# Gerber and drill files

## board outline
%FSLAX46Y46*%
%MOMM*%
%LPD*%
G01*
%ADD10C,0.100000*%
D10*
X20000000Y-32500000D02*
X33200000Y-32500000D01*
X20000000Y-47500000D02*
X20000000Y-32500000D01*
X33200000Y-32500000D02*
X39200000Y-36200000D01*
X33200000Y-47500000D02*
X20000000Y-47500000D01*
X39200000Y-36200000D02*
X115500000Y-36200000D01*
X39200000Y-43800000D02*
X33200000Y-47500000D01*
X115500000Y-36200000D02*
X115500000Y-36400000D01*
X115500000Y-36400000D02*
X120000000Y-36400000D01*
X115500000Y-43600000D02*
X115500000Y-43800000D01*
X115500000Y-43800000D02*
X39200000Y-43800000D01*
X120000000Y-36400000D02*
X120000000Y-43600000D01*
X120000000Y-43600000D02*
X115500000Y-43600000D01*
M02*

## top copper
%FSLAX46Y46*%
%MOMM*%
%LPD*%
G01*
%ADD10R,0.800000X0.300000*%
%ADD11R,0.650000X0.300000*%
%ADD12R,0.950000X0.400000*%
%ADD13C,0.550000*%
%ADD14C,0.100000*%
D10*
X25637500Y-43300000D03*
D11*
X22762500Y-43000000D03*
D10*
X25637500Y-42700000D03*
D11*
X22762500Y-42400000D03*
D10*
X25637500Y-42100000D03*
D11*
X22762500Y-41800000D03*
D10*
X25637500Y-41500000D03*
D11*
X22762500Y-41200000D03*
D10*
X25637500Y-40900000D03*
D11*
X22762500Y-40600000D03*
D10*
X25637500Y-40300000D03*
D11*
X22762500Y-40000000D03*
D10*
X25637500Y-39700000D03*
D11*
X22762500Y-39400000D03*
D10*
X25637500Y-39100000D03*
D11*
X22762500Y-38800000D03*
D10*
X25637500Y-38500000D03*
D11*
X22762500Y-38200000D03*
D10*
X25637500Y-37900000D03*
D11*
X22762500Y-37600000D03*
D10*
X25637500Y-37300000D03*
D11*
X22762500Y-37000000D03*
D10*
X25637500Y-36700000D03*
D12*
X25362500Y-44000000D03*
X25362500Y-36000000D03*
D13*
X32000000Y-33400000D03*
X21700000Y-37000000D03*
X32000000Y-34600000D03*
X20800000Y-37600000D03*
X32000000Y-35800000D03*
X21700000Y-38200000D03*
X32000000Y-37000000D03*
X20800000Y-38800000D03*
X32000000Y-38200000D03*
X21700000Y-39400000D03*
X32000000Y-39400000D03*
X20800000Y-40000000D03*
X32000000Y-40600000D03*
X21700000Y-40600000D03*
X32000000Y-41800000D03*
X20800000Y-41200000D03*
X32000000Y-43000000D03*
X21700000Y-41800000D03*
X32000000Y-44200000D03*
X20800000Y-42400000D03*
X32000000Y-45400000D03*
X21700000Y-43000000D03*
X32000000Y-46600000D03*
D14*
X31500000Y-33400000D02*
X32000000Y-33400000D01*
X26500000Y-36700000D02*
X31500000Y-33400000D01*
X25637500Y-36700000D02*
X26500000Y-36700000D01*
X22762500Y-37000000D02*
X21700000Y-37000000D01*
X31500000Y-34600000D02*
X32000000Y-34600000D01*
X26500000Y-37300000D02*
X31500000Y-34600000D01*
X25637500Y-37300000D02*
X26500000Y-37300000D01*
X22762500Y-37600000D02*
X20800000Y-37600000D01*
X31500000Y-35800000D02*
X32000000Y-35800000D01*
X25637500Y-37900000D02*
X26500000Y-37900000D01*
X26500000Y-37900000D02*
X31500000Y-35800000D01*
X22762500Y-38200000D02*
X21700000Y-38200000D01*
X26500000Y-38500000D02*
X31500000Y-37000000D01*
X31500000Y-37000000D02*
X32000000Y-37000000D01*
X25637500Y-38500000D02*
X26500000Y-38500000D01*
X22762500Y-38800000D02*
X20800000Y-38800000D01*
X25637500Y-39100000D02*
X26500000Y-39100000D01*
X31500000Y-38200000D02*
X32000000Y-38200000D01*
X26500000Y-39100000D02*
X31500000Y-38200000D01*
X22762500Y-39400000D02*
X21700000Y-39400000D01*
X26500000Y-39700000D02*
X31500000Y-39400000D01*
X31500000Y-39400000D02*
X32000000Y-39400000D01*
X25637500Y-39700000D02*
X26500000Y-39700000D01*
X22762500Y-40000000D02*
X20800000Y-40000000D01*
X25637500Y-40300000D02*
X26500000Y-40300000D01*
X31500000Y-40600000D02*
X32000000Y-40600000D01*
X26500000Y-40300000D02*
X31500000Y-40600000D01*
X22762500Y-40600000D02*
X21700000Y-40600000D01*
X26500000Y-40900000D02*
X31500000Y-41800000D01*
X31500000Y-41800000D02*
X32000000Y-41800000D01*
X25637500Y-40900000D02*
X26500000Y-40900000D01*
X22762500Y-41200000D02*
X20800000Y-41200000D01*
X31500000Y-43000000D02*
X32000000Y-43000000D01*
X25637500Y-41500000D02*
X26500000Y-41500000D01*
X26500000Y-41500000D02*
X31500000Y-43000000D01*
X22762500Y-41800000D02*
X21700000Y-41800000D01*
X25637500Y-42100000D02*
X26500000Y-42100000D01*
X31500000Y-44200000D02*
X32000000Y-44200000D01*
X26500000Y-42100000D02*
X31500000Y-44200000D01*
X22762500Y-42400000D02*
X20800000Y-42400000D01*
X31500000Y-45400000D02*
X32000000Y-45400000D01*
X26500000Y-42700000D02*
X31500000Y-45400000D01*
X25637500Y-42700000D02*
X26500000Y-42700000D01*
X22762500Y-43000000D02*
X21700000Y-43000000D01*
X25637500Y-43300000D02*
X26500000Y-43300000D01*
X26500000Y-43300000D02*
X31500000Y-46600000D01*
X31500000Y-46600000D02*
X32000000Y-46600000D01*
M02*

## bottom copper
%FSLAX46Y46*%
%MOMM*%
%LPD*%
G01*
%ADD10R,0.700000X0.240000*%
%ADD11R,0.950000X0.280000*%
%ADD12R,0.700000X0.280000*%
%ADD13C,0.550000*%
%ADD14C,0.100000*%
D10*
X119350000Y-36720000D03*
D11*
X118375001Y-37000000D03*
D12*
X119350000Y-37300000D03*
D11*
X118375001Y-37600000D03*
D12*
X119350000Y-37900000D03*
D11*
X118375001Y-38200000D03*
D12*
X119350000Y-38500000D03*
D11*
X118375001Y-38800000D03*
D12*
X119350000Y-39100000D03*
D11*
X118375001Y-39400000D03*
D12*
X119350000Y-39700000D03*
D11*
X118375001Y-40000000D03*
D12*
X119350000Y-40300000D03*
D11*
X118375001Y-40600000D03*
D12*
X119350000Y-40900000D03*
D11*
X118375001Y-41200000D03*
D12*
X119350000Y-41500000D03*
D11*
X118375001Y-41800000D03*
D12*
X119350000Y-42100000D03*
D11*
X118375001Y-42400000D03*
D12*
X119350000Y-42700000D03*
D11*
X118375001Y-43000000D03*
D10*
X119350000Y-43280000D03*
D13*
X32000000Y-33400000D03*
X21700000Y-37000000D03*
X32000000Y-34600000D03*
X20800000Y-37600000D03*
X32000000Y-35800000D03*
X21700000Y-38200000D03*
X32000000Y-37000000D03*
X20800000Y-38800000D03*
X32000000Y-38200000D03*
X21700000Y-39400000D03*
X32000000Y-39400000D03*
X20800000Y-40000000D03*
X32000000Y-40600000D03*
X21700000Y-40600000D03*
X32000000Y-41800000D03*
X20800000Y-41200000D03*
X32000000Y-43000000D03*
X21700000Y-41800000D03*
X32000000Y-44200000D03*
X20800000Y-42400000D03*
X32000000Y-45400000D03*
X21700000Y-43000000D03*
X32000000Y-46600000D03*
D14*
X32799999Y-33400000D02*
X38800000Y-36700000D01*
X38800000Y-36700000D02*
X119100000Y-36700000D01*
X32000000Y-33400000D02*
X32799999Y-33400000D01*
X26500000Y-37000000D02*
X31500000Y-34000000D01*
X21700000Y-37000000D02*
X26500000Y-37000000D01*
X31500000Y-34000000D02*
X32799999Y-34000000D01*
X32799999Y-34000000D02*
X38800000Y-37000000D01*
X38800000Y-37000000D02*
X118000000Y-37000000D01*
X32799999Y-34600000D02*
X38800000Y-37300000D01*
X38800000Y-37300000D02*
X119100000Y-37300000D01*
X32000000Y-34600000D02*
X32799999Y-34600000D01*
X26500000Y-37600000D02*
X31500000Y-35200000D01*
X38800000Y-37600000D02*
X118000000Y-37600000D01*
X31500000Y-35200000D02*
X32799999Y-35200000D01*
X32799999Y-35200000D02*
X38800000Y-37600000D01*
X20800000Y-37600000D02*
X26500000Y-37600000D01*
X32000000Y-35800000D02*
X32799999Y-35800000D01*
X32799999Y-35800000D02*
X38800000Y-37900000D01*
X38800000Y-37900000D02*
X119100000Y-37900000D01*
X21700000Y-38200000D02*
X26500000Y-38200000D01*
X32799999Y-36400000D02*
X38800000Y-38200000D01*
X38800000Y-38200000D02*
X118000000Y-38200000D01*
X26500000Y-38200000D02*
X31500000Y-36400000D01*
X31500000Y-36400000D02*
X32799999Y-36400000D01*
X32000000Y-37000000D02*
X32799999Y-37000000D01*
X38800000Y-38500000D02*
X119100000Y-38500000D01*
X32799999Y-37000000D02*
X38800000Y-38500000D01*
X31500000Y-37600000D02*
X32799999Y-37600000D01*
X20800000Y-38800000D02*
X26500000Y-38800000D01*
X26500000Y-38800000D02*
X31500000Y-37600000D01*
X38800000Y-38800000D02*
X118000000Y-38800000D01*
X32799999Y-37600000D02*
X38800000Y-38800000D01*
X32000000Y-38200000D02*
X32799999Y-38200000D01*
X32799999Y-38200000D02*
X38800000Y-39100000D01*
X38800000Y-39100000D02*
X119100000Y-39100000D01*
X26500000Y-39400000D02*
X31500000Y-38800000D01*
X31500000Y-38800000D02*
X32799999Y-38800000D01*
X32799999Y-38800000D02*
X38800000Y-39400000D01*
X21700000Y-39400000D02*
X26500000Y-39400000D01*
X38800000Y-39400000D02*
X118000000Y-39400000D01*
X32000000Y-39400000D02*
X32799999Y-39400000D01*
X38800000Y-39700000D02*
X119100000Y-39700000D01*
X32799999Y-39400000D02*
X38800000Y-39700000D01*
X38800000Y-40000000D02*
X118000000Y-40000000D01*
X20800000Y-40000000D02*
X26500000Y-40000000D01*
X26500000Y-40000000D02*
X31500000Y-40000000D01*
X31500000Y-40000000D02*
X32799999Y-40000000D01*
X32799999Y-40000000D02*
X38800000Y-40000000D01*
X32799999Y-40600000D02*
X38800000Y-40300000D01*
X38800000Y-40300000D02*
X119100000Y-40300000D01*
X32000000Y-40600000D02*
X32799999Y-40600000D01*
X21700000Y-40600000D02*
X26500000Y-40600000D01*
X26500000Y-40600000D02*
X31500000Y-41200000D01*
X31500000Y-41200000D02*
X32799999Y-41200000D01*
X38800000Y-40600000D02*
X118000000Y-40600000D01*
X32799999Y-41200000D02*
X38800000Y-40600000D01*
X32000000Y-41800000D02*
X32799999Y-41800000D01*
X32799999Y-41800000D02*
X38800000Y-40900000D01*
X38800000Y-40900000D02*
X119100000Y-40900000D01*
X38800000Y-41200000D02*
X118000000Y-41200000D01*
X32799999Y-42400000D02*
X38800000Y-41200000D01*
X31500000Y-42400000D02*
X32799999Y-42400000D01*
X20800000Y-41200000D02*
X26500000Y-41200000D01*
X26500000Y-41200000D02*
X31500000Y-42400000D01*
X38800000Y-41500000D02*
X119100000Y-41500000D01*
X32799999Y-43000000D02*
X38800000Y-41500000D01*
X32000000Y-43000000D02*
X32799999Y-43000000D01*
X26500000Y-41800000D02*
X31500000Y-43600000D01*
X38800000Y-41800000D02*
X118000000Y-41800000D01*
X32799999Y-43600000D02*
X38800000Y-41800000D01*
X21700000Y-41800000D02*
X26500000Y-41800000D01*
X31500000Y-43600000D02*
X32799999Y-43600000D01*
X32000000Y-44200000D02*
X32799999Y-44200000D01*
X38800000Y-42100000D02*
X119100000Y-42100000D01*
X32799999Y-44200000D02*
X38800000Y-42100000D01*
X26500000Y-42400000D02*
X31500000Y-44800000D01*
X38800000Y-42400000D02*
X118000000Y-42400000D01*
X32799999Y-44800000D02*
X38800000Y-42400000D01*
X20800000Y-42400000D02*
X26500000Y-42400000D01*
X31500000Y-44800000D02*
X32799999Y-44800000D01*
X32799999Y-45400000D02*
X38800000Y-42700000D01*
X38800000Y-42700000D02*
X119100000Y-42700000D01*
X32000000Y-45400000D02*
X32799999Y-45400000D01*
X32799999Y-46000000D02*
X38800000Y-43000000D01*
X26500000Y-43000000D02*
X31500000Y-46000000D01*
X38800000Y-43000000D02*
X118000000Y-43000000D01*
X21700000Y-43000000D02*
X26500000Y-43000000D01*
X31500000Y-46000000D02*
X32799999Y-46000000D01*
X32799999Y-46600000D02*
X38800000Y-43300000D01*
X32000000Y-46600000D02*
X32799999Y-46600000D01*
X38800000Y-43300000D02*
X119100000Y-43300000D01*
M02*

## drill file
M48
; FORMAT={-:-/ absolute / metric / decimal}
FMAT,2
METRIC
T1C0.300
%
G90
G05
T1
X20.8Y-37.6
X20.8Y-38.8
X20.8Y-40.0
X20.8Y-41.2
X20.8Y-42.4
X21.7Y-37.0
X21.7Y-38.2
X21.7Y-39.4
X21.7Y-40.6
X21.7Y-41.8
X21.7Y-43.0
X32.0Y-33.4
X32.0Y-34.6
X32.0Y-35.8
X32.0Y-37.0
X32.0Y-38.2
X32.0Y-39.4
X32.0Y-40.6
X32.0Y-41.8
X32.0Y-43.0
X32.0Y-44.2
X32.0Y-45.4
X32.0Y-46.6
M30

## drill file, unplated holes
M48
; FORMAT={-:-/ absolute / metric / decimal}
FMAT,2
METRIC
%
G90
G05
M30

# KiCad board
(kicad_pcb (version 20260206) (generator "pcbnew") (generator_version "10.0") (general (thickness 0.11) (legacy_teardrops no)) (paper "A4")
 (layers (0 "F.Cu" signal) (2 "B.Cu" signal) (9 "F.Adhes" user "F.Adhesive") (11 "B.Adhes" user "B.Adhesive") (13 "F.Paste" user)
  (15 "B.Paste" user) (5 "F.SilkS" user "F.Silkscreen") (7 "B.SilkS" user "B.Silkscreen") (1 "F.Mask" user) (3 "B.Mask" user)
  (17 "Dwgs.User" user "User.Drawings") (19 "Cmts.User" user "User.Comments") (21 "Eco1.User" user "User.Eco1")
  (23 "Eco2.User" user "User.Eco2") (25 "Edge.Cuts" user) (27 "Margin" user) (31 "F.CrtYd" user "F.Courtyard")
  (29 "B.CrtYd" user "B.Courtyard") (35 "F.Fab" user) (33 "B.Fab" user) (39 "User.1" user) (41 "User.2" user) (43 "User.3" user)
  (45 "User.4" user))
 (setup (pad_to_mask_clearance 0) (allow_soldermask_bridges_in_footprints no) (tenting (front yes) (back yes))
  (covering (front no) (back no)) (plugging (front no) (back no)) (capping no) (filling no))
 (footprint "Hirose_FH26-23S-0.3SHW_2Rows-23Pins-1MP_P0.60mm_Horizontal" (layer "F.Cu") (at 24.2375 40 180)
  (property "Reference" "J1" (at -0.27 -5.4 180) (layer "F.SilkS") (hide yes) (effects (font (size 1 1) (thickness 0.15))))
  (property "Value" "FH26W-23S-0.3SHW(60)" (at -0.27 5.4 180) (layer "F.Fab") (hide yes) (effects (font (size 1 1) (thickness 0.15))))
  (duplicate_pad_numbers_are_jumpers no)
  (pad "1" smd rect (at -1.4 -3.3 180) (size 0.8 0.3) (layers "F.Cu" "F.Mask" "F.Paste") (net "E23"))
  (pad "2" smd rect (at 1.475 -3 180) (size 0.65 0.3) (layers "F.Cu" "F.Mask" "F.Paste") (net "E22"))
  (pad "3" smd rect (at -1.4 -2.7 180) (size 0.8 0.3) (layers "F.Cu" "F.Mask" "F.Paste") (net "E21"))
  (pad "4" smd rect (at 1.475 -2.4 180) (size 0.65 0.3) (layers "F.Cu" "F.Mask" "F.Paste") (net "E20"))
  (pad "5" smd rect (at -1.4 -2.1 180) (size 0.8 0.3) (layers "F.Cu" "F.Mask" "F.Paste") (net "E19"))
  (pad "6" smd rect (at 1.475 -1.8 180) (size 0.65 0.3) (layers "F.Cu" "F.Mask" "F.Paste") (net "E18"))
  (pad "7" smd rect (at -1.4 -1.5 180) (size 0.8 0.3) (layers "F.Cu" "F.Mask" "F.Paste") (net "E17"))
  (pad "8" smd rect (at 1.475 -1.2 180) (size 0.65 0.3) (layers "F.Cu" "F.Mask" "F.Paste") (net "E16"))
  (pad "9" smd rect (at -1.4 -0.9 180) (size 0.8 0.3) (layers "F.Cu" "F.Mask" "F.Paste") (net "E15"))
  (pad "10" smd rect (at 1.475 -0.6 180) (size 0.65 0.3) (layers "F.Cu" "F.Mask" "F.Paste") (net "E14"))
  (pad "11" smd rect (at -1.4 -0.3 180) (size 0.8 0.3) (layers "F.Cu" "F.Mask" "F.Paste") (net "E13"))
  (pad "12" smd rect (at 1.475 0 180) (size 0.65 0.3) (layers "F.Cu" "F.Mask" "F.Paste") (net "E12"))
  (pad "13" smd rect (at -1.4 0.3 180) (size 0.8 0.3) (layers "F.Cu" "F.Mask" "F.Paste") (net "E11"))
  (pad "14" smd rect (at 1.475 0.6 180) (size 0.65 0.3) (layers "F.Cu" "F.Mask" "F.Paste") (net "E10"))
  (pad "15" smd rect (at -1.4 0.9 180) (size 0.8 0.3) (layers "F.Cu" "F.Mask" "F.Paste") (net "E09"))
  (pad "16" smd rect (at 1.475 1.2 180) (size 0.65 0.3) (layers "F.Cu" "F.Mask" "F.Paste") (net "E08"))
  (pad "17" smd rect (at -1.4 1.5 180) (size 0.8 0.3) (layers "F.Cu" "F.Mask" "F.Paste") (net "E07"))
  (pad "18" smd rect (at 1.475 1.8 180) (size 0.65 0.3) (layers "F.Cu" "F.Mask" "F.Paste") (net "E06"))
  (pad "19" smd rect (at -1.4 2.1 180) (size 0.8 0.3) (layers "F.Cu" "F.Mask" "F.Paste") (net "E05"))
  (pad "20" smd rect (at 1.475 2.4 180) (size 0.65 0.3) (layers "F.Cu" "F.Mask" "F.Paste") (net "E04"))
  (pad "21" smd rect (at -1.4 2.7 180) (size 0.8 0.3) (layers "F.Cu" "F.Mask" "F.Paste") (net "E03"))
  (pad "22" smd rect (at 1.475 3 180) (size 0.65 0.3) (layers "F.Cu" "F.Mask" "F.Paste") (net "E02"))
  (pad "23" smd rect (at -1.4 3.3 180) (size 0.8 0.3) (layers "F.Cu" "F.Mask" "F.Paste") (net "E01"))
  (pad "MP" smd rect (at -1.125 -4 180) (size 0.95 0.4) (layers "F.Cu" "F.Mask" "F.Paste"))
  (pad "MP" smd rect (at -1.125 4 180) (size 0.95 0.4) (layers "F.Cu" "F.Mask" "F.Paste")))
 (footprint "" (layer "B.Cu") (at 118.6 40 180)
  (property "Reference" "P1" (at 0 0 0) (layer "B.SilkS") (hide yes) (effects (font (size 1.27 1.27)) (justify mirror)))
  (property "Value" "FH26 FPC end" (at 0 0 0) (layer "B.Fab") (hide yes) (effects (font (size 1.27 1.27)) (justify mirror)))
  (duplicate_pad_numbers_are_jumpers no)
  (pad "1" smd rect (at -0.75 3.28 180) (size 0.7 0.24) (layers "B.Cu" "B.Mask") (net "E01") (thermal_bridge_angle 45))
  (pad "2" smd rect (at 0.224999 3 180) (size 0.95 0.28) (layers "B.Cu" "B.Mask") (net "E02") (thermal_bridge_angle 45))
  (pad "3" smd rect (at -0.75 2.7 180) (size 0.7 0.28) (layers "B.Cu" "B.Mask") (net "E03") (thermal_bridge_angle 45))
  (pad "4" smd rect (at 0.224999 2.4 180) (size 0.95 0.28) (layers "B.Cu" "B.Mask") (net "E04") (thermal_bridge_angle 45))
  (pad "5" smd rect (at -0.75 2.1 180) (size 0.7 0.28) (layers "B.Cu" "B.Mask") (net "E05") (thermal_bridge_angle 45))
  (pad "6" smd rect (at 0.224999 1.8 180) (size 0.95 0.28) (layers "B.Cu" "B.Mask") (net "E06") (thermal_bridge_angle 45))
  (pad "7" smd rect (at -0.75 1.5 180) (size 0.7 0.28) (layers "B.Cu" "B.Mask") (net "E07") (thermal_bridge_angle 45))
  (pad "8" smd rect (at 0.224999 1.2 180) (size 0.95 0.28) (layers "B.Cu" "B.Mask") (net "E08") (thermal_bridge_angle 45))
  (pad "9" smd rect (at -0.75 0.9 180) (size 0.7 0.28) (layers "B.Cu" "B.Mask") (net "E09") (thermal_bridge_angle 45))
  (pad "10" smd rect (at 0.224999 0.6 180) (size 0.95 0.28) (layers "B.Cu" "B.Mask") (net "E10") (thermal_bridge_angle 45))
  (pad "11" smd rect (at -0.75 0.3 180) (size 0.7 0.28) (layers "B.Cu" "B.Mask") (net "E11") (thermal_bridge_angle 45))
  (pad "12" smd rect (at 0.224999 0 180) (size 0.95 0.28) (layers "B.Cu" "B.Mask") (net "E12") (thermal_bridge_angle 45))
  (pad "13" smd rect (at -0.75 -0.3 180) (size 0.7 0.28) (layers "B.Cu" "B.Mask") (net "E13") (thermal_bridge_angle 45))
  (pad "14" smd rect (at 0.224999 -0.6 180) (size 0.95 0.28) (layers "B.Cu" "B.Mask") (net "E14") (thermal_bridge_angle 45))
  (pad "15" smd rect (at -0.75 -0.9 180) (size 0.7 0.28) (layers "B.Cu" "B.Mask") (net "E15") (thermal_bridge_angle 45))
  (pad "16" smd rect (at 0.224999 -1.2 180) (size 0.95 0.28) (layers "B.Cu" "B.Mask") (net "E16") (thermal_bridge_angle 45))
  (pad "17" smd rect (at -0.75 -1.5 180) (size 0.7 0.28) (layers "B.Cu" "B.Mask") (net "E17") (thermal_bridge_angle 45))
  (pad "18" smd rect (at 0.224999 -1.8 180) (size 0.95 0.28) (layers "B.Cu" "B.Mask") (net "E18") (thermal_bridge_angle 45))
  (pad "19" smd rect (at -0.75 -2.1 180) (size 0.7 0.28) (layers "B.Cu" "B.Mask") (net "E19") (thermal_bridge_angle 45))
  (pad "20" smd rect (at 0.224999 -2.4 180) (size 0.95 0.28) (layers "B.Cu" "B.Mask") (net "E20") (thermal_bridge_angle 45))
  (pad "21" smd rect (at -0.75 -2.7 180) (size 0.7 0.28) (layers "B.Cu" "B.Mask") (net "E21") (thermal_bridge_angle 45))
  (pad "22" smd rect (at 0.224999 -3 180) (size 0.95 0.28) (layers "B.Cu" "B.Mask") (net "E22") (thermal_bridge_angle 45))
  (pad "23" smd rect (at -0.75 -3.28 180) (size 0.7 0.24) (layers "B.Cu" "B.Mask") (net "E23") (thermal_bridge_angle 45)))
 (gr_line (start 20 32.5) (end 33.2 32.5) (stroke (width 0.1) (type default)) (layer "Edge.Cuts"))
 (gr_line (start 20 47.5) (end 20 32.5) (stroke (width 0.1) (type default)) (layer "Edge.Cuts"))
 (gr_line (start 33.2 32.5) (end 39.2 36.2) (stroke (width 0.1) (type default)) (layer "Edge.Cuts"))
 (gr_line (start 33.2 47.5) (end 20 47.5) (stroke (width 0.1) (type default)) (layer "Edge.Cuts"))
 (gr_line (start 39.2 36.2) (end 115.5 36.2) (stroke (width 0.1) (type default)) (layer "Edge.Cuts"))
 (gr_line (start 39.2 43.8) (end 33.2 47.5) (stroke (width 0.1) (type default)) (layer "Edge.Cuts"))
 (gr_line (start 115.5 36.2) (end 115.5 36.4) (stroke (width 0.1) (type default)) (layer "Edge.Cuts"))
 (gr_line (start 115.5 36.4) (end 120 36.4) (stroke (width 0.1) (type default)) (layer "Edge.Cuts"))
 (gr_line (start 115.5 43.6) (end 115.5 43.8) (stroke (width 0.1) (type default)) (layer "Edge.Cuts"))
 (gr_line (start 115.5 43.8) (end 39.2 43.8) (stroke (width 0.1) (type default)) (layer "Edge.Cuts"))
 (gr_line (start 120 36.4) (end 120 43.6) (stroke (width 0.1) (type default)) (layer "Edge.Cuts"))
 (gr_line (start 120 43.6) (end 115.5 43.6) (stroke (width 0.1) (type default)) (layer "Edge.Cuts"))
 (segment (start 31.5 33.4) (end 32 33.4) (width 0.1) (layer "F.Cu") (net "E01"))
 (segment (start 26.5 36.7) (end 31.5 33.4) (width 0.1) (layer "F.Cu") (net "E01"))
 (segment (start 25.6375 36.7) (end 26.5 36.7) (width 0.1) (layer "F.Cu") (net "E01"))
 (via (at 32 33.4) (size 0.55) (drill 0.3) (layers "F.Cu" "B.Cu") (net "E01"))
 (segment (start 32.799999 33.4) (end 38.8 36.7) (width 0.1) (layer "B.Cu") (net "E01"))
 (segment (start 38.8 36.7) (end 119.1 36.7) (width 0.1) (layer "B.Cu") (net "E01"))
 (segment (start 32 33.4) (end 32.799999 33.4) (width 0.1) (layer "B.Cu") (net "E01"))
 (segment (start 22.7625 37) (end 21.7 37) (width 0.1) (layer "F.Cu") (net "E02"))
 (via (at 21.7 37) (size 0.55) (drill 0.3) (layers "F.Cu" "B.Cu") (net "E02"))
 (segment (start 26.5 37) (end 31.5 34) (width 0.1) (layer "B.Cu") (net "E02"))
 (segment (start 21.7 37) (end 26.5 37) (width 0.1) (layer "B.Cu") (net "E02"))
 (segment (start 31.5 34) (end 32.799999 34) (width 0.1) (layer "B.Cu") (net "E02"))
 (segment (start 32.799999 34) (end 38.8 37) (width 0.1) (layer "B.Cu") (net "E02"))
 (segment (start 38.8 37) (end 118 37) (width 0.1) (layer "B.Cu") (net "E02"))
 (segment (start 31.5 34.6) (end 32 34.6) (width 0.1) (layer "F.Cu") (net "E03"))
 (segment (start 26.5 37.3) (end 31.5 34.6) (width 0.1) (layer "F.Cu") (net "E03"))
 (segment (start 25.6375 37.3) (end 26.5 37.3) (width 0.1) (layer "F.Cu") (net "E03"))
 (via (at 32 34.6) (size 0.55) (drill 0.3) (layers "F.Cu" "B.Cu") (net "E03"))
 (segment (start 32.799999 34.6) (end 38.8 37.3) (width 0.1) (layer "B.Cu") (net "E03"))
 (segment (start 38.8 37.3) (end 119.1 37.3) (width 0.1) (layer "B.Cu") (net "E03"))
 (segment (start 32 34.6) (end 32.799999 34.6) (width 0.1) (layer "B.Cu") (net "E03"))
 (segment (start 22.7625 37.6) (end 20.8 37.6) (width 0.1) (layer "F.Cu") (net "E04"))
 (via (at 20.8 37.6) (size 0.55) (drill 0.3) (layers "F.Cu" "B.Cu") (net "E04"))
 (segment (start 26.5 37.6) (end 31.5 35.2) (width 0.1) (layer "B.Cu") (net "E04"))
 (segment (start 38.8 37.6) (end 118 37.6) (width 0.1) (layer "B.Cu") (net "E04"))
 (segment (start 31.5 35.2) (end 32.799999 35.2) (width 0.1) (layer "B.Cu") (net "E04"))
 (segment (start 32.799999 35.2) (end 38.8 37.6) (width 0.1) (layer "B.Cu") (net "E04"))
 (segment (start 20.8 37.6) (end 26.5 37.6) (width 0.1) (layer "B.Cu") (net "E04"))
 (segment (start 31.5 35.8) (end 32 35.8) (width 0.1) (layer "F.Cu") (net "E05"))
 (segment (start 25.6375 37.9) (end 26.5 37.9) (width 0.1) (layer "F.Cu") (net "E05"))
 (segment (start 26.5 37.9) (end 31.5 35.8) (width 0.1) (layer "F.Cu") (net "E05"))
 (via (at 32 35.8) (size 0.55) (drill 0.3) (layers "F.Cu" "B.Cu") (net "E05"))
 (segment (start 32 35.8) (end 32.799999 35.8) (width 0.1) (layer "B.Cu") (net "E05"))
 (segment (start 32.799999 35.8) (end 38.8 37.9) (width 0.1) (layer "B.Cu") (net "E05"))
 (segment (start 38.8 37.9) (end 119.1 37.9) (width 0.1) (layer "B.Cu") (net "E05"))
 (segment (start 22.7625 38.2) (end 21.7 38.2) (width 0.1) (layer "F.Cu") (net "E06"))
 (via (at 21.7 38.2) (size 0.55) (drill 0.3) (layers "F.Cu" "B.Cu") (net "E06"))
 (segment (start 21.7 38.2) (end 26.5 38.2) (width 0.1) (layer "B.Cu") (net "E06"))
 (segment (start 32.799999 36.4) (end 38.8 38.2) (width 0.1) (layer "B.Cu") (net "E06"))
 (segment (start 38.8 38.2) (end 118 38.2) (width 0.1) (layer "B.Cu") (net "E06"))
 (segment (start 26.5 38.2) (end 31.5 36.4) (width 0.1) (layer "B.Cu") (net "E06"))
 (segment (start 31.5 36.4) (end 32.799999 36.4) (width 0.1) (layer "B.Cu") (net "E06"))
 (segment (start 26.5 38.5) (end 31.5 37) (width 0.1) (layer "F.Cu") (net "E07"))
 (segment (start 31.5 37) (end 32 37) (width 0.1) (layer "F.Cu") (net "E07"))
 (segment (start 25.6375 38.5) (end 26.5 38.5) (width 0.1) (layer "F.Cu") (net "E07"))
 (via (at 32 37) (size 0.55) (drill 0.3) (layers "F.Cu" "B.Cu") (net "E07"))
 (segment (start 32 37) (end 32.799999 37) (width 0.1) (layer "B.Cu") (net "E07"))
 (segment (start 38.8 38.5) (end 119.1 38.5) (width 0.1) (layer "B.Cu") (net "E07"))
 (segment (start 32.799999 37) (end 38.8 38.5) (width 0.1) (layer "B.Cu") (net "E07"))
 (segment (start 22.7625 38.8) (end 20.8 38.8) (width 0.1) (layer "F.Cu") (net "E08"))
 (via (at 20.8 38.8) (size 0.55) (drill 0.3) (layers "F.Cu" "B.Cu") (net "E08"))
 (segment (start 31.5 37.6) (end 32.799999 37.6) (width 0.1) (layer "B.Cu") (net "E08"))
 (segment (start 20.8 38.8) (end 26.5 38.8) (width 0.1) (layer "B.Cu") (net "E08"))
 (segment (start 26.5 38.8) (end 31.5 37.6) (width 0.1) (layer "B.Cu") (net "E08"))
 (segment (start 38.8 38.8) (end 118 38.8) (width 0.1) (layer "B.Cu") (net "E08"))
 (segment (start 32.799999 37.6) (end 38.8 38.8) (width 0.1) (layer "B.Cu") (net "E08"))
 (segment (start 25.6375 39.1) (end 26.5 39.1) (width 0.1) (layer "F.Cu") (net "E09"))
 (segment (start 31.5 38.2) (end 32 38.2) (width 0.1) (layer "F.Cu") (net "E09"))
 (segment (start 26.5 39.1) (end 31.5 38.2) (width 0.1) (layer "F.Cu") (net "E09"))
 (via (at 32 38.2) (size 0.55) (drill 0.3) (layers "F.Cu" "B.Cu") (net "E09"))
 (segment (start 32 38.2) (end 32.799999 38.2) (width 0.1) (layer "B.Cu") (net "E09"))
 (segment (start 32.799999 38.2) (end 38.8 39.1) (width 0.1) (layer "B.Cu") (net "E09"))
 (segment (start 38.8 39.1) (end 119.1 39.1) (width 0.1) (layer "B.Cu") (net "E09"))
 (segment (start 22.7625 39.4) (end 21.7 39.4) (width 0.1) (layer "F.Cu") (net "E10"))
 (via (at 21.7 39.4) (size 0.55) (drill 0.3) (layers "F.Cu" "B.Cu") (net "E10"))
 (segment (start 26.5 39.4) (end 31.5 38.8) (width 0.1) (layer "B.Cu") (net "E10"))
 (segment (start 31.5 38.8) (end 32.799999 38.8) (width 0.1) (layer "B.Cu") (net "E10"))
 (segment (start 32.799999 38.8) (end 38.8 39.4) (width 0.1) (layer "B.Cu") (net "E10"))
 (segment (start 21.7 39.4) (end 26.5 39.4) (width 0.1) (layer "B.Cu") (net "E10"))
 (segment (start 38.8 39.4) (end 118 39.4) (width 0.1) (layer "B.Cu") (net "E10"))
 (segment (start 26.5 39.7) (end 31.5 39.4) (width 0.1) (layer "F.Cu") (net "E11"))
 (segment (start 31.5 39.4) (end 32 39.4) (width 0.1) (layer "F.Cu") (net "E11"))
 (segment (start 25.6375 39.7) (end 26.5 39.7) (width 0.1) (layer "F.Cu") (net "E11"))
 (via (at 32 39.4) (size 0.55) (drill 0.3) (layers "F.Cu" "B.Cu") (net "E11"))
 (segment (start 32 39.4) (end 32.799999 39.4) (width 0.1) (layer "B.Cu") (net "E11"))
 (segment (start 38.8 39.7) (end 119.1 39.7) (width 0.1) (layer "B.Cu") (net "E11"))
 (segment (start 32.799999 39.4) (end 38.8 39.7) (width 0.1) (layer "B.Cu") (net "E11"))
 (segment (start 22.7625 40) (end 20.8 40) (width 0.1) (layer "F.Cu") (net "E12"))
 (via (at 20.8 40) (size 0.55) (drill 0.3) (layers "F.Cu" "B.Cu") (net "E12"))
 (segment (start 38.8 40) (end 118 40) (width 0.1) (layer "B.Cu") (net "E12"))
 (segment (start 20.8 40) (end 26.5 40) (width 0.1) (layer "B.Cu") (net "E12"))
 (segment (start 26.5 40) (end 31.5 40) (width 0.1) (layer "B.Cu") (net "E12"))
 (segment (start 31.5 40) (end 32.799999 40) (width 0.1) (layer "B.Cu") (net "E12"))
 (segment (start 32.799999 40) (end 38.8 40) (width 0.1) (layer "B.Cu") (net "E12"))
 (segment (start 25.6375 40.3) (end 26.5 40.3) (width 0.1) (layer "F.Cu") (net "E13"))
 (segment (start 31.5 40.6) (end 32 40.6) (width 0.1) (layer "F.Cu") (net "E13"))
 (segment (start 26.5 40.3) (end 31.5 40.6) (width 0.1) (layer "F.Cu") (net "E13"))
 (via (at 32 40.6) (size 0.55) (drill 0.3) (layers "F.Cu" "B.Cu") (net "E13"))
 (segment (start 32.799999 40.6) (end 38.8 40.3) (width 0.1) (layer "B.Cu") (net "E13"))
 (segment (start 38.8 40.3) (end 119.1 40.3) (width 0.1) (layer "B.Cu") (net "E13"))
 (segment (start 32 40.6) (end 32.799999 40.6) (width 0.1) (layer "B.Cu") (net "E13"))
 (segment (start 22.7625 40.6) (end 21.7 40.6) (width 0.1) (layer "F.Cu") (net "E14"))
 (via (at 21.7 40.6) (size 0.55) (drill 0.3) (layers "F.Cu" "B.Cu") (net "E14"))
 (segment (start 21.7 40.6) (end 26.5 40.6) (width 0.1) (layer "B.Cu") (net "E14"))
 (segment (start 26.5 40.6) (end 31.5 41.2) (width 0.1) (layer "B.Cu") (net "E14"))
 (segment (start 31.5 41.2) (end 32.799999 41.2) (width 0.1) (layer "B.Cu") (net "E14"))
 (segment (start 38.8 40.6) (end 118 40.6) (width 0.1) (layer "B.Cu") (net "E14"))
 (segment (start 32.799999 41.2) (end 38.8 40.6) (width 0.1) (layer "B.Cu") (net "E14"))
 (segment (start 26.5 40.9) (end 31.5 41.8) (width 0.1) (layer "F.Cu") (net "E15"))
 (segment (start 31.5 41.8) (end 32 41.8) (width 0.1) (layer "F.Cu") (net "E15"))
 (segment (start 25.6375 40.9) (end 26.5 40.9) (width 0.1) (layer "F.Cu") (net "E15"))
 (via (at 32 41.8) (size 0.55) (drill 0.3) (layers "F.Cu" "B.Cu") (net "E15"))
 (segment (start 32 41.8) (end 32.799999 41.8) (width 0.1) (layer "B.Cu") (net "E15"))
 (segment (start 32.799999 41.8) (end 38.8 40.9) (width 0.1) (layer "B.Cu") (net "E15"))
 (segment (start 38.8 40.9) (end 119.1 40.9) (width 0.1) (layer "B.Cu") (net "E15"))
 (segment (start 22.7625 41.2) (end 20.8 41.2) (width 0.1) (layer "F.Cu") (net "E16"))
 (via (at 20.8 41.2) (size 0.55) (drill 0.3) (layers "F.Cu" "B.Cu") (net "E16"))
 (segment (start 38.8 41.2) (end 118 41.2) (width 0.1) (layer "B.Cu") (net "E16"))
 (segment (start 32.799999 42.4) (end 38.8 41.2) (width 0.1) (layer "B.Cu") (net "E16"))
 (segment (start 31.5 42.4) (end 32.799999 42.4) (width 0.1) (layer "B.Cu") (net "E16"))
 (segment (start 20.8 41.2) (end 26.5 41.2) (width 0.1) (layer "B.Cu") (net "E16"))
 (segment (start 26.5 41.2) (end 31.5 42.4) (width 0.1) (layer "B.Cu") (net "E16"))
 (segment (start 31.5 43) (end 32 43) (width 0.1) (layer "F.Cu") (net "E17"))
 (segment (start 25.6375 41.5) (end 26.5 41.5) (width 0.1) (layer "F.Cu") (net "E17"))
 (segment (start 26.5 41.5) (end 31.5 43) (width 0.1) (layer "F.Cu") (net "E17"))
 (via (at 32 43) (size 0.55) (drill 0.3) (layers "F.Cu" "B.Cu") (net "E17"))
 (segment (start 38.8 41.5) (end 119.1 41.5) (width 0.1) (layer "B.Cu") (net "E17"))
 (segment (start 32.799999 43) (end 38.8 41.5) (width 0.1) (layer "B.Cu") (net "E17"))
 (segment (start 32 43) (end 32.799999 43) (width 0.1) (layer "B.Cu") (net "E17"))
 (segment (start 22.7625 41.8) (end 21.7 41.8) (width 0.1) (layer "F.Cu") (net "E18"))
 (via (at 21.7 41.8) (size 0.55) (drill 0.3) (layers "F.Cu" "B.Cu") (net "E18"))
 (segment (start 26.5 41.8) (end 31.5 43.6) (width 0.1) (layer "B.Cu") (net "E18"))
 (segment (start 38.8 41.8) (end 118 41.8) (width 0.1) (layer "B.Cu") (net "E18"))
 (segment (start 32.799999 43.6) (end 38.8 41.8) (width 0.1) (layer "B.Cu") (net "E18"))
 (segment (start 21.7 41.8) (end 26.5 41.8) (width 0.1) (layer "B.Cu") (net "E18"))
 (segment (start 31.5 43.6) (end 32.799999 43.6) (width 0.1) (layer "B.Cu") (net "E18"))
 (segment (start 25.6375 42.1) (end 26.5 42.1) (width 0.1) (layer "F.Cu") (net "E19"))
 (segment (start 31.5 44.2) (end 32 44.2) (width 0.1) (layer "F.Cu") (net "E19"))
 (segment (start 26.5 42.1) (end 31.5 44.2) (width 0.1) (layer "F.Cu") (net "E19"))
 (via (at 32 44.2) (size 0.55) (drill 0.3) (layers "F.Cu" "B.Cu") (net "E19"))
 (segment (start 32 44.2) (end 32.799999 44.2) (width 0.1) (layer "B.Cu") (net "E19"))
 (segment (start 38.8 42.1) (end 119.1 42.1) (width 0.1) (layer "B.Cu") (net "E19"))
 (segment (start 32.799999 44.2) (end 38.8 42.1) (width 0.1) (layer "B.Cu") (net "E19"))
 (segment (start 22.7625 42.4) (end 20.8 42.4) (width 0.1) (layer "F.Cu") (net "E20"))
 (via (at 20.8 42.4) (size 0.55) (drill 0.3) (layers "F.Cu" "B.Cu") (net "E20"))
 (segment (start 26.5 42.4) (end 31.5 44.8) (width 0.1) (layer "B.Cu") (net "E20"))
 (segment (start 38.8 42.4) (end 118 42.4) (width 0.1) (layer "B.Cu") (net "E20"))
 (segment (start 32.799999 44.8) (end 38.8 42.4) (width 0.1) (layer "B.Cu") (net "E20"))
 (segment (start 20.8 42.4) (end 26.5 42.4) (width 0.1) (layer "B.Cu") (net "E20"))
 (segment (start 31.5 44.8) (end 32.799999 44.8) (width 0.1) (layer "B.Cu") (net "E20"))
 (segment (start 31.5 45.4) (end 32 45.4) (width 0.1) (layer "F.Cu") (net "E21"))
 (segment (start 26.5 42.7) (end 31.5 45.4) (width 0.1) (layer "F.Cu") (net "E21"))
 (segment (start 25.6375 42.7) (end 26.5 42.7) (width 0.1) (layer "F.Cu") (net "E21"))
 (via (at 32 45.4) (size 0.55) (drill 0.3) (layers "F.Cu" "B.Cu") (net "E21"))
 (segment (start 32.799999 45.4) (end 38.8 42.7) (width 0.1) (layer "B.Cu") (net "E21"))
 (segment (start 38.8 42.7) (end 119.1 42.7) (width 0.1) (layer "B.Cu") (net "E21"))
 (segment (start 32 45.4) (end 32.799999 45.4) (width 0.1) (layer "B.Cu") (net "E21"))
 (segment (start 22.7625 43) (end 21.7 43) (width 0.1) (layer "F.Cu") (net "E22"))
 (via (at 21.7 43) (size 0.55) (drill 0.3) (layers "F.Cu" "B.Cu") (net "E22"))
 (segment (start 32.799999 46) (end 38.8 43) (width 0.1) (layer "B.Cu") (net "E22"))
 (segment (start 26.5 43) (end 31.5 46) (width 0.1) (layer "B.Cu") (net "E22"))
 (segment (start 38.8 43) (end 118 43) (width 0.1) (layer "B.Cu") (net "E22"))
 (segment (start 21.7 43) (end 26.5 43) (width 0.1) (layer "B.Cu") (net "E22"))
 (segment (start 31.5 46) (end 32.799999 46) (width 0.1) (layer "B.Cu") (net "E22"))
 (segment (start 25.6375 43.3) (end 26.5 43.3) (width 0.1) (layer "F.Cu") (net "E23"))
 (segment (start 26.5 43.3) (end 31.5 46.6) (width 0.1) (layer "F.Cu") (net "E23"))
 (segment (start 31.5 46.6) (end 32 46.6) (width 0.1) (layer "F.Cu") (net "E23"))
 (via (at 32 46.6) (size 0.55) (drill 0.3) (layers "F.Cu" "B.Cu") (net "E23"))
 (segment (start 32.799999 46.6) (end 38.8 43.3) (width 0.1) (layer "B.Cu") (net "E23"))
 (segment (start 32 46.6) (end 32.799999 46.6) (width 0.1) (layer "B.Cu") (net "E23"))
 (segment (start 38.8 43.3) (end 119.1 43.3) (width 0.1) (layer "B.Cu") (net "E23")))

